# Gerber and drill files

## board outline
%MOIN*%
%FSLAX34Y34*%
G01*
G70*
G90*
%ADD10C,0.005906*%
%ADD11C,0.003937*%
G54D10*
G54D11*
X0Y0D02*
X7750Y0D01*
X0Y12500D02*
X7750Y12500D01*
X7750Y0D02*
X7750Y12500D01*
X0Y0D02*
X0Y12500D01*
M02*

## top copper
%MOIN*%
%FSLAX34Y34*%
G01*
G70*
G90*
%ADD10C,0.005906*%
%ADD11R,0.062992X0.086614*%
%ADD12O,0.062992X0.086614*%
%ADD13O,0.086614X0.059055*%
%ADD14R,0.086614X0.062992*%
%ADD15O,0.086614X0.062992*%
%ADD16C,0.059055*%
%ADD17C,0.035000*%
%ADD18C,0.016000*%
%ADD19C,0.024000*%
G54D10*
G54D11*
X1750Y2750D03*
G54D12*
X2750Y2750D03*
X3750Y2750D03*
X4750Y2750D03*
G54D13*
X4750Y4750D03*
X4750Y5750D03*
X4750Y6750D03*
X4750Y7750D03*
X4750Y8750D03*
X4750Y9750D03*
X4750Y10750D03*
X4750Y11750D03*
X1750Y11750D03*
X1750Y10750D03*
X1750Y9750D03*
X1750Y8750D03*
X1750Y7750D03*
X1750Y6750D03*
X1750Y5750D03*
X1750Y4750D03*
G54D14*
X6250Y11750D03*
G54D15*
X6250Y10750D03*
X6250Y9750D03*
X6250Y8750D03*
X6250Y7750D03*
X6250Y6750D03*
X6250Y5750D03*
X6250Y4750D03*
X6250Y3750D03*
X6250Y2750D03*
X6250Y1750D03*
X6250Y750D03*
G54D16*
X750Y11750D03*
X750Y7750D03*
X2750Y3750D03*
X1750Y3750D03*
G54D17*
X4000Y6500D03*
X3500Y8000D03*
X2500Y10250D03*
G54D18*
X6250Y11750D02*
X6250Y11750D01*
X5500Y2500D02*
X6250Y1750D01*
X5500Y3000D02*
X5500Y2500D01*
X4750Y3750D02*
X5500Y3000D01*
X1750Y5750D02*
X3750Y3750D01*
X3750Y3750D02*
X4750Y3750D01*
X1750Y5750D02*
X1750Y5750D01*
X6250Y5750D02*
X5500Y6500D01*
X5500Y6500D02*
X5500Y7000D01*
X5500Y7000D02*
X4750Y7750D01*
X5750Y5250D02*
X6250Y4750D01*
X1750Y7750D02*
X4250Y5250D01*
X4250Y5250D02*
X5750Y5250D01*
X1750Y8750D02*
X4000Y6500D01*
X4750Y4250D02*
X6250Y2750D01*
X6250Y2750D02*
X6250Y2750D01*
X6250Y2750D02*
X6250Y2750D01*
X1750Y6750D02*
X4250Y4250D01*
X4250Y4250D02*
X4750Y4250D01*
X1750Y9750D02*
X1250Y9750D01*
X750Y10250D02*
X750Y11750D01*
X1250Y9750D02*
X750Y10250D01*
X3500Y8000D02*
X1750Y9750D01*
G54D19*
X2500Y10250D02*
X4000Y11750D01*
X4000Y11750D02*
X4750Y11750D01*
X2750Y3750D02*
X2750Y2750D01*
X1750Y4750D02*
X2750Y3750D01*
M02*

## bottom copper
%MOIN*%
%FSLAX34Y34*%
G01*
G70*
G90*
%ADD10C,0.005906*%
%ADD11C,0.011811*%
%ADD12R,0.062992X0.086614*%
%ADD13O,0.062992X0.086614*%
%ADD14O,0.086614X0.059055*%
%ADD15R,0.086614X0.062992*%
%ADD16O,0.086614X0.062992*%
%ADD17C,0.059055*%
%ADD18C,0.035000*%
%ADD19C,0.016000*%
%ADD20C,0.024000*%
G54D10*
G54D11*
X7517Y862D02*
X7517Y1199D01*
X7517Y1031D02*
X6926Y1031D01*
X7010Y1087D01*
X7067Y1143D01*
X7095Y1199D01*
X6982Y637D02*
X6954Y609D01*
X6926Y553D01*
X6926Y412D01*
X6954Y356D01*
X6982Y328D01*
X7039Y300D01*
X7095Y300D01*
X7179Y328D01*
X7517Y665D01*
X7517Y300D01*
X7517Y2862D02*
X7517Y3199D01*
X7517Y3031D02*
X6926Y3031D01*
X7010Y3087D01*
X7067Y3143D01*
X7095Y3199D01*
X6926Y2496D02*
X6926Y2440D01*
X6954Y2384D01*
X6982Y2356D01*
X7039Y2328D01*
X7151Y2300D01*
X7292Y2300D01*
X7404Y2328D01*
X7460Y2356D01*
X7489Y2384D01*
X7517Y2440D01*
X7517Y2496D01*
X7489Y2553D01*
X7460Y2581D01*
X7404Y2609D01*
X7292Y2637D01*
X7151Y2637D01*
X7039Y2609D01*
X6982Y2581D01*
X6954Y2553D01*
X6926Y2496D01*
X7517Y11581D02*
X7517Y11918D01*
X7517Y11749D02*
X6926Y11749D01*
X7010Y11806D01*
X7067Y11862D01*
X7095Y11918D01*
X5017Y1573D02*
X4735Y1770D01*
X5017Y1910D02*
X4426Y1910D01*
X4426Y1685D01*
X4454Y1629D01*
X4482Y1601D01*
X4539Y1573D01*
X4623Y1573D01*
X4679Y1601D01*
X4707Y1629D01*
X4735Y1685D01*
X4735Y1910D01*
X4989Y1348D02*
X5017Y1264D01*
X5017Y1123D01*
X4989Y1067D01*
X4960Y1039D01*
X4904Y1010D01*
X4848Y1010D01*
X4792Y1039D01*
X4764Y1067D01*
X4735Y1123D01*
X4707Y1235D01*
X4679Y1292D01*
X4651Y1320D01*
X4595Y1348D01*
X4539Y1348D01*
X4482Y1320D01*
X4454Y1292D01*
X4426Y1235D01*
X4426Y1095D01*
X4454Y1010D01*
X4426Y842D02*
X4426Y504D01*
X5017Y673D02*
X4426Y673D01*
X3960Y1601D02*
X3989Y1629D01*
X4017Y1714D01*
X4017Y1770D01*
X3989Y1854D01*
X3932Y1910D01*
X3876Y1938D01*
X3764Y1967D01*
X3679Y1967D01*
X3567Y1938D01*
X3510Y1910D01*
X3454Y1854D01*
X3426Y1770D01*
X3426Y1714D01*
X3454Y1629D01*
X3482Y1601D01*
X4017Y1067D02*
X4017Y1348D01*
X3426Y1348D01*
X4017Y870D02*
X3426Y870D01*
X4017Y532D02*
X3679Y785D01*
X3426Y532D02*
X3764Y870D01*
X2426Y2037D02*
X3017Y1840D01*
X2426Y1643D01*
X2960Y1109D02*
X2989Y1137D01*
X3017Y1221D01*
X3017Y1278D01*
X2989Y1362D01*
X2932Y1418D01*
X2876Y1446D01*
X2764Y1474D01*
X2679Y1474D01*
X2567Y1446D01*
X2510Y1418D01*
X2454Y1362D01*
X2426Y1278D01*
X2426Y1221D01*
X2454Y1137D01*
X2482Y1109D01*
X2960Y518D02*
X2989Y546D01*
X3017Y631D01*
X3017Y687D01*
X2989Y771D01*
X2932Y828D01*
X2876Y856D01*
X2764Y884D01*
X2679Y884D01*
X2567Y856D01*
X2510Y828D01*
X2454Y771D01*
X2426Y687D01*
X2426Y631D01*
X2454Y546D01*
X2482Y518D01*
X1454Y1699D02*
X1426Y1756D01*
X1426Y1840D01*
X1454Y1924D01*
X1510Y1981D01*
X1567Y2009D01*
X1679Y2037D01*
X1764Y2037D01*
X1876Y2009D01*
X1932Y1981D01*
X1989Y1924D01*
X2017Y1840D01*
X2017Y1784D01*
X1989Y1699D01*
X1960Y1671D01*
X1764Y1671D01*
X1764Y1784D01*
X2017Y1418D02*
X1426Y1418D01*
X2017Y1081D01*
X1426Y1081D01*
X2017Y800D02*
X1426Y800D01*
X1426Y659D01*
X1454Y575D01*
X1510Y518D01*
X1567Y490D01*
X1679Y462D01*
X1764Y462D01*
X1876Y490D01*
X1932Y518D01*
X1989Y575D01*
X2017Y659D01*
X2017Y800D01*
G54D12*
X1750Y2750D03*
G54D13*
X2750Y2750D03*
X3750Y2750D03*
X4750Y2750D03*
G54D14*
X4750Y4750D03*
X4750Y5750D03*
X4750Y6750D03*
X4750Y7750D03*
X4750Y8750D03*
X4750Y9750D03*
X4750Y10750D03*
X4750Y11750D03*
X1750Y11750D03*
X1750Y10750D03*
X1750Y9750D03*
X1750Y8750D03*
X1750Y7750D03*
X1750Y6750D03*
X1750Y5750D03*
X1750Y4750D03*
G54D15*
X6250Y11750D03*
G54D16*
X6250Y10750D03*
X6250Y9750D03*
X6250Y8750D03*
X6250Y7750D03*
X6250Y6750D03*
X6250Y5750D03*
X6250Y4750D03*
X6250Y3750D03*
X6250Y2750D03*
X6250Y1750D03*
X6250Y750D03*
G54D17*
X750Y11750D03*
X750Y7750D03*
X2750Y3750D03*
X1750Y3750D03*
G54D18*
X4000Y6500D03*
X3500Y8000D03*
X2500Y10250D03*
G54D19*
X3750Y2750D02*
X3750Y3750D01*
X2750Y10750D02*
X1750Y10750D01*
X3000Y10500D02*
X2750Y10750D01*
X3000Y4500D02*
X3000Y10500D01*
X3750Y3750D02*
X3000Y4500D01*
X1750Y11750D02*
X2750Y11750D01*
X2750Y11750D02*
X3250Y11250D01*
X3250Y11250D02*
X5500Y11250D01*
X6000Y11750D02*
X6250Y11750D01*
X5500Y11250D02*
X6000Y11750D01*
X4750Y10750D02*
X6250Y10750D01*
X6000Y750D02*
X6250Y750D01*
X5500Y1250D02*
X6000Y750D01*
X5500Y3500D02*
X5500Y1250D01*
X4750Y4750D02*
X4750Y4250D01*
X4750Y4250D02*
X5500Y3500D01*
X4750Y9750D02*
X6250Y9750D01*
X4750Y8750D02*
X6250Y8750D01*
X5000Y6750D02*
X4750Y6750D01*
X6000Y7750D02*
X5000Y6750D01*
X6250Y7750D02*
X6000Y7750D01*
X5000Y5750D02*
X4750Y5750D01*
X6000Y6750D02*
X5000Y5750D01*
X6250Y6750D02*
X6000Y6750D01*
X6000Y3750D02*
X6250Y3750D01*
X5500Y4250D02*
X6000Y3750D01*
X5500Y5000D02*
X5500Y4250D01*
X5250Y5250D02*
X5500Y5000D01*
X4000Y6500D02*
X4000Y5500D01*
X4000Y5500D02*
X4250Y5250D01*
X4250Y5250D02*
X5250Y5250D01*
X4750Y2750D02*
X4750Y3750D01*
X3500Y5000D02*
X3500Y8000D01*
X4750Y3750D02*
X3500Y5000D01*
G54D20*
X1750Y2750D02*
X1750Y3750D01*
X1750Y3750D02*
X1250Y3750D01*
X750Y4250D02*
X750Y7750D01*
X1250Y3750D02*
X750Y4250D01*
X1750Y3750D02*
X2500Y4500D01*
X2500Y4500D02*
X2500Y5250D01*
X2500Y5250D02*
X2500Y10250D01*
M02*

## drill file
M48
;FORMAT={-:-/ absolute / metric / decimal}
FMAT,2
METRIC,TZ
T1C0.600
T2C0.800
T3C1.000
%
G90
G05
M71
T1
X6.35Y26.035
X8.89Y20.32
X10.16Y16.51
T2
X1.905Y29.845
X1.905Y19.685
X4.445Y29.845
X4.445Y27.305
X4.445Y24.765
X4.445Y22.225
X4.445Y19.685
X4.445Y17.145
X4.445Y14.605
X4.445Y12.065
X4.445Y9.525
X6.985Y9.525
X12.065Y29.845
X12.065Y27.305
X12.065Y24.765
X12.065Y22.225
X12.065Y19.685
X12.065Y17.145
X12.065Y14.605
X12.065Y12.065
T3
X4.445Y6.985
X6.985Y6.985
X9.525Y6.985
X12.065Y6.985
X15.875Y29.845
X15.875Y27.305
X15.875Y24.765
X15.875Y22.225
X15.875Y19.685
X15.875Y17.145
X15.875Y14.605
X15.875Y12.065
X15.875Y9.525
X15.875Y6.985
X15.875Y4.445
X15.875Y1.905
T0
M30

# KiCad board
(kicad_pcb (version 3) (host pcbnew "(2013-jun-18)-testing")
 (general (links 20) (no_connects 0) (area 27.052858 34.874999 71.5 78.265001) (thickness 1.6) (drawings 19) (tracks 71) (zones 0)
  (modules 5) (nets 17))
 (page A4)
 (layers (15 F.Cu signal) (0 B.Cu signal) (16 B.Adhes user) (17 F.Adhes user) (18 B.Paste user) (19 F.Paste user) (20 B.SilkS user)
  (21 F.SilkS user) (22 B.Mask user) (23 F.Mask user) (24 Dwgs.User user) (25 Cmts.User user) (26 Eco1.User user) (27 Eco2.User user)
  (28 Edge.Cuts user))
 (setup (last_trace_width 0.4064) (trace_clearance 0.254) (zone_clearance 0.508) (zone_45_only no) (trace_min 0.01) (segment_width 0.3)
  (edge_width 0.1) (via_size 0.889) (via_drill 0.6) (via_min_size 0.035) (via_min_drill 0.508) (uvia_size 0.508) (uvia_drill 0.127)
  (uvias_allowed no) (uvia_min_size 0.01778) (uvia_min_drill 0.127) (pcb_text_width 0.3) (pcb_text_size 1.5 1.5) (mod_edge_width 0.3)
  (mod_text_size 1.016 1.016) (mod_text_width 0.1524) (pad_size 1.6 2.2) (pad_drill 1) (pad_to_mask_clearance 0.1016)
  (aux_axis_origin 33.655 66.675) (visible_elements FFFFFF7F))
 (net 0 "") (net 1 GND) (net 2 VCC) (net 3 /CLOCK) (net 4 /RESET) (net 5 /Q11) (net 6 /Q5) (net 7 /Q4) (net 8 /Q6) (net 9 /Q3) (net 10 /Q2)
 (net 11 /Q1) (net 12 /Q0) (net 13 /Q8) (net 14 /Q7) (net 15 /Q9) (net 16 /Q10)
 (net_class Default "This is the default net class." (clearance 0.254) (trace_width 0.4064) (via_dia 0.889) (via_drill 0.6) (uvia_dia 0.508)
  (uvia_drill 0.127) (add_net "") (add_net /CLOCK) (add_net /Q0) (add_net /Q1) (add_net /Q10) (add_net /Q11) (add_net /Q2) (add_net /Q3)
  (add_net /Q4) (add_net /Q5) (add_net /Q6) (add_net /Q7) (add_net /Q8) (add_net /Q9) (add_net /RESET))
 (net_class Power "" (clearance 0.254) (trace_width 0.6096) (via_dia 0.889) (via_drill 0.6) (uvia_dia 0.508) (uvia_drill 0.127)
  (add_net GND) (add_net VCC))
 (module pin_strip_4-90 (layer F.Cu) (at 41.91 59.69)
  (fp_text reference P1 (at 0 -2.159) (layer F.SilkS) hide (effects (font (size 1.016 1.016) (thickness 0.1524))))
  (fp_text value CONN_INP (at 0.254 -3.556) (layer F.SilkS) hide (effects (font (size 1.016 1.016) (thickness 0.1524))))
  (pad 1 thru_hole rect (at -3.81 0) (size 1.6 2.2) (drill 1) (layers *.Cu *.Mask F.SilkS) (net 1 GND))
  (pad 2 thru_hole oval (at -1.27 0) (size 1.6 2.2) (drill 1) (layers *.Cu *.Mask F.SilkS) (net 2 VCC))
  (pad 3 thru_hole oval (at 1.27 0) (size 1.6 2.2) (drill 1) (layers *.Cu *.Mask F.SilkS) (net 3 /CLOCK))
  (pad 4 thru_hole oval (at 3.81 0) (size 1.6 2.2) (drill 1) (layers *.Cu *.Mask F.SilkS) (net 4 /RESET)))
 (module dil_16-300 (layer F.Cu) (at 41.91 45.72 90)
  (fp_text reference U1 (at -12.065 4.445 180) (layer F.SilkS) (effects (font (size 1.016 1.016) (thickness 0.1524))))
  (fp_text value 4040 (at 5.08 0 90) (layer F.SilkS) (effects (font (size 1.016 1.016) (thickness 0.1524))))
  (pad 1 thru_hole oval (at -8.89 3.81 90) (size 1.5 2.2) (drill 0.8) (layers *.Cu *.Mask F.SilkS) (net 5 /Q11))
  (pad 2 thru_hole oval (at -6.35 3.81 90) (size 1.5 2.2) (drill 0.8) (layers *.Cu *.Mask F.SilkS) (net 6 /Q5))
  (pad 3 thru_hole oval (at -3.81 3.81 90) (size 1.5 2.2) (drill 0.8) (layers *.Cu *.Mask F.SilkS) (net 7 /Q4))
  (pad 4 thru_hole oval (at -1.27 3.81 90) (size 1.5 2.2) (drill 0.8) (layers *.Cu *.Mask F.SilkS) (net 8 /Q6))
  (pad 5 thru_hole oval (at 1.27 3.81 90) (size 1.5 2.2) (drill 0.8) (layers *.Cu *.Mask F.SilkS) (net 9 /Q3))
  (pad 6 thru_hole oval (at 3.81 3.81 90) (size 1.5 2.2) (drill 0.8) (layers *.Cu *.Mask F.SilkS) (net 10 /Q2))
  (pad 7 thru_hole oval (at 6.35 3.81 90) (size 1.5 2.2) (drill 0.8) (layers *.Cu *.Mask F.SilkS) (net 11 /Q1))
  (pad 8 thru_hole oval (at 8.89 3.81 90) (size 1.5 2.2) (drill 0.8) (layers *.Cu *.Mask F.SilkS) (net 1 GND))
  (pad 9 thru_hole oval (at 8.89 -3.81 90) (size 1.5 2.2) (drill 0.8) (layers *.Cu *.Mask F.SilkS) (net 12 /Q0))
  (pad 10 thru_hole oval (at 6.35 -3.81 90) (size 1.5 2.2) (drill 0.8) (layers *.Cu *.Mask F.SilkS) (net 3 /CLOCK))
  (pad 11 thru_hole oval (at 3.81 -3.81 90) (size 1.5 2.2) (drill 0.8) (layers *.Cu *.Mask F.SilkS) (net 4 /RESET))
  (pad 12 thru_hole oval (at 1.27 -3.81 90) (size 1.5 2.2) (drill 0.8) (layers *.Cu *.Mask F.SilkS) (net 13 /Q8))
  (pad 13 thru_hole oval (at -1.27 -3.81 90) (size 1.5 2.2) (drill 0.8) (layers *.Cu *.Mask F.SilkS) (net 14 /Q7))
  (pad 14 thru_hole oval (at -3.81 -3.81 90) (size 1.5 2.2) (drill 0.8) (layers *.Cu *.Mask F.SilkS) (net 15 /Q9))
  (pad 15 thru_hole oval (at -6.35 -3.81 90) (size 1.5 2.2) (drill 0.8) (layers *.Cu *.Mask F.SilkS) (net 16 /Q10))
  (pad 16 thru_hole oval (at -8.89 -3.81 90) (size 1.5 2.2) (drill 0.8) (layers *.Cu *.Mask F.SilkS) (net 2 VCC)))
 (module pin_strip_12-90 (layer F.Cu) (at 49.53 50.8 90)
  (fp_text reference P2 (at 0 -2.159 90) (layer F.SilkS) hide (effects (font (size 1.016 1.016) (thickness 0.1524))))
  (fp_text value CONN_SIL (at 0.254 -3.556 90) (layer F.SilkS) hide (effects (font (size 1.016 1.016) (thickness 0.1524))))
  (pad 1 thru_hole rect (at 13.97 0 270) (size 1.6 2.2) (drill 1) (layers *.Cu *.Mask F.SilkS) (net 12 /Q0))
  (pad 2 thru_hole oval (at 11.43 0 270) (size 1.6 2.2) (drill 1) (layers *.Cu *.Mask F.SilkS) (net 11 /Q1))
  (pad 3 thru_hole oval (at 8.89 0 270) (size 1.6 2.2) (drill 1) (layers *.Cu *.Mask F.SilkS) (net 10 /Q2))
  (pad 4 thru_hole oval (at 6.35 0 270) (size 1.6 2.2) (drill 1) (layers *.Cu *.Mask F.SilkS) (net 9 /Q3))
  (pad 5 thru_hole oval (at 3.81 0 270) (size 1.6 2.2) (drill 1) (layers *.Cu *.Mask F.SilkS) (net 7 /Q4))
  (pad 6 thru_hole oval (at 1.27 0 270) (size 1.6 2.2) (drill 1) (layers *.Cu *.Mask F.SilkS) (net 6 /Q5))
  (pad 7 thru_hole oval (at -1.27 0 270) (size 1.6 2.2) (drill 1) (layers *.Cu *.Mask F.SilkS) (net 8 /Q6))
  (pad 8 thru_hole oval (at -3.81 0 270) (size 1.6 2.2) (drill 1) (layers *.Cu *.Mask F.SilkS) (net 14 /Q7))
  (pad 9 thru_hole oval (at -6.35 0 270) (size 1.6 2.2) (drill 1) (layers *.Cu *.Mask F.SilkS) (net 13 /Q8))
  (pad 10 thru_hole oval (at -8.89 0 270) (size 1.6 2.2) (drill 1) (layers *.Cu *.Mask F.SilkS) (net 15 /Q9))
  (pad 11 thru_hole oval (at -11.43 0 270) (size 1.6 2.2) (drill 1) (layers *.Cu *.Mask F.SilkS) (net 16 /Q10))
  (pad 12 thru_hole oval (at -13.97 0 270) (size 1.6 2.2) (drill 1) (layers *.Cu *.Mask F.SilkS) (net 5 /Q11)))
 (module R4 (layer F.Cu) (at 35.56 41.91 270) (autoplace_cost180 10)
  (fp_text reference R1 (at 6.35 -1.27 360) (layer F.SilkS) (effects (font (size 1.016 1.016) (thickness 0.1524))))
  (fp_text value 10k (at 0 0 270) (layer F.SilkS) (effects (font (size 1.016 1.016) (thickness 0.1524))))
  (pad 1 thru_hole circle (at -5.08 0 270) (size 1.5 1.5) (drill 0.8) (layers *.Cu *.Mask F.SilkS) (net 4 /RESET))
  (pad 2 thru_hole circle (at 5.08 0 270) (size 1.5 1.5) (drill 0.8) (layers *.Cu *.Mask F.SilkS) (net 1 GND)))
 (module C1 (layer F.Cu) (at 39.37 57.15 180)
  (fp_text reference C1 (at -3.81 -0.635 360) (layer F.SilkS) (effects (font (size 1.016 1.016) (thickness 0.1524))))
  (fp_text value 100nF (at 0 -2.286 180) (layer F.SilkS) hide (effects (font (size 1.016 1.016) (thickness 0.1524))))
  (pad 1 thru_hole circle (at -1.27 0 180) (size 1.5 1.5) (drill 0.8) (layers *.Cu *.Mask F.SilkS) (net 2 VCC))
  (pad 2 thru_hole circle (at 1.27 0 180) (size 1.5 1.5) (drill 0.8) (layers *.Cu *.Mask F.SilkS) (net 1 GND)))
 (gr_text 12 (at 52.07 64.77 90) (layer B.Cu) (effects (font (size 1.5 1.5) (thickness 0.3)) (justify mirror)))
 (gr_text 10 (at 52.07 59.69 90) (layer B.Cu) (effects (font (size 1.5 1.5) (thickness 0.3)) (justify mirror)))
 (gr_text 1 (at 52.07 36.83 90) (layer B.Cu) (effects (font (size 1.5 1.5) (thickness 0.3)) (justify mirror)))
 (gr_line (start 33.655 66.675) (end 53.34 66.675) (angle 90) (layer Edge.Cuts) (width 0.1))
 (gr_line (start 33.655 34.925) (end 53.34 34.925) (angle 90) (layer Edge.Cuts) (width 0.1))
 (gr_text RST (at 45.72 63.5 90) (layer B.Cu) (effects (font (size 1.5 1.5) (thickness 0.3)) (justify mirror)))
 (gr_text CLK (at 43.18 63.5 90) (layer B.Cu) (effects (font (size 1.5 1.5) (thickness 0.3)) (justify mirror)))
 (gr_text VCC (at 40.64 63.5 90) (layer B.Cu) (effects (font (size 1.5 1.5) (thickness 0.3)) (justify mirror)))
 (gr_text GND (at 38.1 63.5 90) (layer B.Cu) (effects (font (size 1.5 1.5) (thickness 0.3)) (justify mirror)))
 (gr_line (start 53.34 66.675) (end 53.34 34.925) (angle 90) (layer Edge.Cuts) (width 0.1))
 (gr_line (start 33.655 66.675) (end 33.655 34.925) (angle 90) (layer Edge.Cuts) (width 0.1))
 (segment (start 43.18 59.69) (end 43.18 57.15) (width 0.4064) (layer B.Cu) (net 3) (status 10))
 (segment (start 40.64 39.37) (end 38.1 39.37) (width 0.4064) (layer B.Cu) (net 3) (status 20))
 (segment (start 41.275 40.005) (end 40.64 39.37) (width 0.4064) (layer B.Cu) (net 3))
 (segment (start 41.275 55.245) (end 41.275 40.005) (width 0.4064) (layer B.Cu) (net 3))
 (segment (start 43.18 57.15) (end 41.275 55.245) (width 0.4064) (layer B.Cu) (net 3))
 (segment (start 38.1 36.83) (end 40.64 36.83) (width 0.4064) (layer B.Cu) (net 12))
 (segment (start 40.64 36.83) (end 41.91 38.1) (width 0.4064) (layer B.Cu) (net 12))
 (segment (start 41.91 38.1) (end 47.625 38.1) (width 0.4064) (layer B.Cu) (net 12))
 (segment (start 48.895 36.83) (end 49.53 36.83) (width 0.4064) (layer B.Cu) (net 12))
 (segment (start 47.625 38.1) (end 48.895 36.83) (width 0.4064) (layer B.Cu) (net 12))
 (segment (start 49.53 36.83) (end 49.53 36.83) (width 0.4064) (layer F.Cu) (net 12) (status 30))
 (segment (start 45.72 39.37) (end 49.53 39.37) (width 0.4064) (layer B.Cu) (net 11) (status 20))
 (segment (start 47.625 60.325) (end 49.53 62.23) (width 0.4064) (layer F.Cu) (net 16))
 (segment (start 47.625 59.055) (end 47.625 60.325) (width 0.4064) (layer F.Cu) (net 16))
 (segment (start 45.72 57.15) (end 47.625 59.055) (width 0.4064) (layer F.Cu) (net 16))
 (segment (start 38.1 52.07) (end 43.18 57.15) (width 0.4064) (layer F.Cu) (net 16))
 (segment (start 43.18 57.15) (end 45.72 57.15) (width 0.4064) (layer F.Cu) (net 16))
 (segment (start 38.1 52.07) (end 38.1 52.07) (width 0.4064) (layer F.Cu) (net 16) (status 10))
 (segment (start 48.895 64.77) (end 49.53 64.77) (width 0.4064) (layer B.Cu) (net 5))
 (segment (start 47.625 63.5) (end 48.895 64.77) (width 0.4064) (layer B.Cu) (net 5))
 (segment (start 47.625 57.785) (end 47.625 63.5) (width 0.4064) (layer B.Cu) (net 5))
 (segment (start 45.72 54.61) (end 45.72 55.88) (width 0.4064) (layer B.Cu) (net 5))
 (segment (start 45.72 55.88) (end 47.625 57.785) (width 0.4064) (layer B.Cu) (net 5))
 (segment (start 45.72 41.91) (end 49.53 41.91) (width 0.4064) (layer B.Cu) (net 10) (status 20))
 (segment (start 45.72 44.45) (end 49.53 44.45) (width 0.4064) (layer B.Cu) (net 9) (status 20))
 (segment (start 46.355 49.53) (end 45.72 49.53) (width 0.4064) (layer B.Cu) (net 7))
 (segment (start 48.895 46.99) (end 46.355 49.53) (width 0.4064) (layer B.Cu) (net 7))
 (segment (start 49.53 46.99) (end 48.895 46.99) (width 0.4064) (layer B.Cu) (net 7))
 (segment (start 46.355 52.07) (end 45.72 52.07) (width 0.4064) (layer B.Cu) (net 6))
 (segment (start 48.895 49.53) (end 46.355 52.07) (width 0.4064) (layer B.Cu) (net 6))
 (segment (start 49.53 49.53) (end 48.895 49.53) (width 0.4064) (layer B.Cu) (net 6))
 (segment (start 49.53 52.07) (end 47.625 50.165) (width 0.4064) (layer F.Cu) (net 8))
 (segment (start 47.625 50.165) (end 47.625 48.895) (width 0.4064) (layer F.Cu) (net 8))
 (segment (start 47.625 48.895) (end 45.72 46.99) (width 0.4064) (layer F.Cu) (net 8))
 (segment (start 48.26 53.34) (end 49.53 54.61) (width 0.4064) (layer F.Cu) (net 14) (status 20))
 (segment (start 38.1 46.99) (end 44.45 53.34) (width 0.4064) (layer F.Cu) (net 14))
 (segment (start 44.45 53.34) (end 48.26 53.34) (width 0.4064) (layer F.Cu) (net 14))
 (segment (start 48.895 57.15) (end 49.53 57.15) (width 0.4064) (layer B.Cu) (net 13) (status 30))
 (segment (start 47.625 55.88) (end 48.895 57.15) (width 0.4064) (layer B.Cu) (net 13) (status 20))
 (segment (start 47.625 53.975) (end 47.625 55.88) (width 0.4064) (layer B.Cu) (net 13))
 (segment (start 38.1 44.45) (end 43.815 50.165) (width 0.4064) (layer F.Cu) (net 13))
 (via (at 43.815 50.165) (size 0.889) (layers F.Cu B.Cu) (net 13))
 (segment (start 46.99 53.34) (end 47.625 53.975) (width 0.4064) (layer B.Cu) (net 13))
 (segment (start 43.815 50.165) (end 43.815 52.705) (width 0.4064) (layer B.Cu) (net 13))
 (segment (start 43.815 52.705) (end 44.45 53.34) (width 0.4064) (layer B.Cu) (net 13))
 (segment (start 44.45 53.34) (end 46.99 53.34) (width 0.4064) (layer B.Cu) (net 13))
 (segment (start 45.72 55.88) (end 49.53 59.69) (width 0.4064) (layer F.Cu) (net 15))
 (segment (start 49.53 59.69) (end 49.53 59.69) (width 0.4064) (layer F.Cu) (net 15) (status 30))
 (segment (start 49.53 59.69) (end 49.53 59.69) (width 0.4064) (layer F.Cu) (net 15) (status 30))
 (segment (start 38.1 49.53) (end 44.45 55.88) (width 0.4064) (layer F.Cu) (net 15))
 (segment (start 44.45 55.88) (end 45.72 55.88) (width 0.4064) (layer F.Cu) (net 15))
 (segment (start 38.1 41.91) (end 36.83 41.91) (width 0.4064) (layer F.Cu) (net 4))
 (segment (start 35.56 40.64) (end 35.56 36.83) (width 0.4064) (layer F.Cu) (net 4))
 (segment (start 36.83 41.91) (end 35.56 40.64) (width 0.4064) (layer F.Cu) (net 4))
 (segment (start 45.72 59.69) (end 45.72 57.15) (width 0.4064) (layer B.Cu) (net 4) (status 10))
 (segment (start 42.545 46.355) (end 38.1 41.91) (width 0.4064) (layer F.Cu) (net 4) (status 20))
 (via (at 42.545 46.355) (size 0.889) (layers F.Cu B.Cu) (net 4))
 (segment (start 42.545 53.975) (end 42.545 46.355) (width 0.4064) (layer B.Cu) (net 4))
 (segment (start 45.72 57.15) (end 42.545 53.975) (width 0.4064) (layer B.Cu) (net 4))
 (segment (start 38.1 59.69) (end 38.1 57.15) (width 0.6096) (layer B.Cu) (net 1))
 (segment (start 38.1 57.15) (end 36.83 57.15) (width 0.6096) (layer B.Cu) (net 1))
 (segment (start 35.56 55.88) (end 35.56 46.99) (width 0.6096) (layer B.Cu) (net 1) (status 20))
 (segment (start 36.83 57.15) (end 35.56 55.88) (width 0.6096) (layer B.Cu) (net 1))
 (segment (start 38.1 57.15) (end 40.005 55.245) (width 0.6096) (layer B.Cu) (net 1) (status 10))
 (segment (start 40.005 55.245) (end 40.005 53.34) (width 0.6096) (layer B.Cu) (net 1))
 (segment (start 40.005 40.64) (end 43.815 36.83) (width 0.6096) (layer F.Cu) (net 1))
 (via (at 40.005 40.64) (size 0.889) (layers F.Cu B.Cu) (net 1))
 (segment (start 40.005 53.34) (end 40.005 40.64) (width 0.6096) (layer B.Cu) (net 1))
 (segment (start 43.815 36.83) (end 45.72 36.83) (width 0.6096) (layer F.Cu) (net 1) (status 20))
 (segment (start 40.64 57.15) (end 40.64 59.69) (width 0.6096) (layer F.Cu) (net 2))
 (segment (start 38.1 54.61) (end 40.64 57.15) (width 0.6096) (layer F.Cu) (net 2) (status 30)))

